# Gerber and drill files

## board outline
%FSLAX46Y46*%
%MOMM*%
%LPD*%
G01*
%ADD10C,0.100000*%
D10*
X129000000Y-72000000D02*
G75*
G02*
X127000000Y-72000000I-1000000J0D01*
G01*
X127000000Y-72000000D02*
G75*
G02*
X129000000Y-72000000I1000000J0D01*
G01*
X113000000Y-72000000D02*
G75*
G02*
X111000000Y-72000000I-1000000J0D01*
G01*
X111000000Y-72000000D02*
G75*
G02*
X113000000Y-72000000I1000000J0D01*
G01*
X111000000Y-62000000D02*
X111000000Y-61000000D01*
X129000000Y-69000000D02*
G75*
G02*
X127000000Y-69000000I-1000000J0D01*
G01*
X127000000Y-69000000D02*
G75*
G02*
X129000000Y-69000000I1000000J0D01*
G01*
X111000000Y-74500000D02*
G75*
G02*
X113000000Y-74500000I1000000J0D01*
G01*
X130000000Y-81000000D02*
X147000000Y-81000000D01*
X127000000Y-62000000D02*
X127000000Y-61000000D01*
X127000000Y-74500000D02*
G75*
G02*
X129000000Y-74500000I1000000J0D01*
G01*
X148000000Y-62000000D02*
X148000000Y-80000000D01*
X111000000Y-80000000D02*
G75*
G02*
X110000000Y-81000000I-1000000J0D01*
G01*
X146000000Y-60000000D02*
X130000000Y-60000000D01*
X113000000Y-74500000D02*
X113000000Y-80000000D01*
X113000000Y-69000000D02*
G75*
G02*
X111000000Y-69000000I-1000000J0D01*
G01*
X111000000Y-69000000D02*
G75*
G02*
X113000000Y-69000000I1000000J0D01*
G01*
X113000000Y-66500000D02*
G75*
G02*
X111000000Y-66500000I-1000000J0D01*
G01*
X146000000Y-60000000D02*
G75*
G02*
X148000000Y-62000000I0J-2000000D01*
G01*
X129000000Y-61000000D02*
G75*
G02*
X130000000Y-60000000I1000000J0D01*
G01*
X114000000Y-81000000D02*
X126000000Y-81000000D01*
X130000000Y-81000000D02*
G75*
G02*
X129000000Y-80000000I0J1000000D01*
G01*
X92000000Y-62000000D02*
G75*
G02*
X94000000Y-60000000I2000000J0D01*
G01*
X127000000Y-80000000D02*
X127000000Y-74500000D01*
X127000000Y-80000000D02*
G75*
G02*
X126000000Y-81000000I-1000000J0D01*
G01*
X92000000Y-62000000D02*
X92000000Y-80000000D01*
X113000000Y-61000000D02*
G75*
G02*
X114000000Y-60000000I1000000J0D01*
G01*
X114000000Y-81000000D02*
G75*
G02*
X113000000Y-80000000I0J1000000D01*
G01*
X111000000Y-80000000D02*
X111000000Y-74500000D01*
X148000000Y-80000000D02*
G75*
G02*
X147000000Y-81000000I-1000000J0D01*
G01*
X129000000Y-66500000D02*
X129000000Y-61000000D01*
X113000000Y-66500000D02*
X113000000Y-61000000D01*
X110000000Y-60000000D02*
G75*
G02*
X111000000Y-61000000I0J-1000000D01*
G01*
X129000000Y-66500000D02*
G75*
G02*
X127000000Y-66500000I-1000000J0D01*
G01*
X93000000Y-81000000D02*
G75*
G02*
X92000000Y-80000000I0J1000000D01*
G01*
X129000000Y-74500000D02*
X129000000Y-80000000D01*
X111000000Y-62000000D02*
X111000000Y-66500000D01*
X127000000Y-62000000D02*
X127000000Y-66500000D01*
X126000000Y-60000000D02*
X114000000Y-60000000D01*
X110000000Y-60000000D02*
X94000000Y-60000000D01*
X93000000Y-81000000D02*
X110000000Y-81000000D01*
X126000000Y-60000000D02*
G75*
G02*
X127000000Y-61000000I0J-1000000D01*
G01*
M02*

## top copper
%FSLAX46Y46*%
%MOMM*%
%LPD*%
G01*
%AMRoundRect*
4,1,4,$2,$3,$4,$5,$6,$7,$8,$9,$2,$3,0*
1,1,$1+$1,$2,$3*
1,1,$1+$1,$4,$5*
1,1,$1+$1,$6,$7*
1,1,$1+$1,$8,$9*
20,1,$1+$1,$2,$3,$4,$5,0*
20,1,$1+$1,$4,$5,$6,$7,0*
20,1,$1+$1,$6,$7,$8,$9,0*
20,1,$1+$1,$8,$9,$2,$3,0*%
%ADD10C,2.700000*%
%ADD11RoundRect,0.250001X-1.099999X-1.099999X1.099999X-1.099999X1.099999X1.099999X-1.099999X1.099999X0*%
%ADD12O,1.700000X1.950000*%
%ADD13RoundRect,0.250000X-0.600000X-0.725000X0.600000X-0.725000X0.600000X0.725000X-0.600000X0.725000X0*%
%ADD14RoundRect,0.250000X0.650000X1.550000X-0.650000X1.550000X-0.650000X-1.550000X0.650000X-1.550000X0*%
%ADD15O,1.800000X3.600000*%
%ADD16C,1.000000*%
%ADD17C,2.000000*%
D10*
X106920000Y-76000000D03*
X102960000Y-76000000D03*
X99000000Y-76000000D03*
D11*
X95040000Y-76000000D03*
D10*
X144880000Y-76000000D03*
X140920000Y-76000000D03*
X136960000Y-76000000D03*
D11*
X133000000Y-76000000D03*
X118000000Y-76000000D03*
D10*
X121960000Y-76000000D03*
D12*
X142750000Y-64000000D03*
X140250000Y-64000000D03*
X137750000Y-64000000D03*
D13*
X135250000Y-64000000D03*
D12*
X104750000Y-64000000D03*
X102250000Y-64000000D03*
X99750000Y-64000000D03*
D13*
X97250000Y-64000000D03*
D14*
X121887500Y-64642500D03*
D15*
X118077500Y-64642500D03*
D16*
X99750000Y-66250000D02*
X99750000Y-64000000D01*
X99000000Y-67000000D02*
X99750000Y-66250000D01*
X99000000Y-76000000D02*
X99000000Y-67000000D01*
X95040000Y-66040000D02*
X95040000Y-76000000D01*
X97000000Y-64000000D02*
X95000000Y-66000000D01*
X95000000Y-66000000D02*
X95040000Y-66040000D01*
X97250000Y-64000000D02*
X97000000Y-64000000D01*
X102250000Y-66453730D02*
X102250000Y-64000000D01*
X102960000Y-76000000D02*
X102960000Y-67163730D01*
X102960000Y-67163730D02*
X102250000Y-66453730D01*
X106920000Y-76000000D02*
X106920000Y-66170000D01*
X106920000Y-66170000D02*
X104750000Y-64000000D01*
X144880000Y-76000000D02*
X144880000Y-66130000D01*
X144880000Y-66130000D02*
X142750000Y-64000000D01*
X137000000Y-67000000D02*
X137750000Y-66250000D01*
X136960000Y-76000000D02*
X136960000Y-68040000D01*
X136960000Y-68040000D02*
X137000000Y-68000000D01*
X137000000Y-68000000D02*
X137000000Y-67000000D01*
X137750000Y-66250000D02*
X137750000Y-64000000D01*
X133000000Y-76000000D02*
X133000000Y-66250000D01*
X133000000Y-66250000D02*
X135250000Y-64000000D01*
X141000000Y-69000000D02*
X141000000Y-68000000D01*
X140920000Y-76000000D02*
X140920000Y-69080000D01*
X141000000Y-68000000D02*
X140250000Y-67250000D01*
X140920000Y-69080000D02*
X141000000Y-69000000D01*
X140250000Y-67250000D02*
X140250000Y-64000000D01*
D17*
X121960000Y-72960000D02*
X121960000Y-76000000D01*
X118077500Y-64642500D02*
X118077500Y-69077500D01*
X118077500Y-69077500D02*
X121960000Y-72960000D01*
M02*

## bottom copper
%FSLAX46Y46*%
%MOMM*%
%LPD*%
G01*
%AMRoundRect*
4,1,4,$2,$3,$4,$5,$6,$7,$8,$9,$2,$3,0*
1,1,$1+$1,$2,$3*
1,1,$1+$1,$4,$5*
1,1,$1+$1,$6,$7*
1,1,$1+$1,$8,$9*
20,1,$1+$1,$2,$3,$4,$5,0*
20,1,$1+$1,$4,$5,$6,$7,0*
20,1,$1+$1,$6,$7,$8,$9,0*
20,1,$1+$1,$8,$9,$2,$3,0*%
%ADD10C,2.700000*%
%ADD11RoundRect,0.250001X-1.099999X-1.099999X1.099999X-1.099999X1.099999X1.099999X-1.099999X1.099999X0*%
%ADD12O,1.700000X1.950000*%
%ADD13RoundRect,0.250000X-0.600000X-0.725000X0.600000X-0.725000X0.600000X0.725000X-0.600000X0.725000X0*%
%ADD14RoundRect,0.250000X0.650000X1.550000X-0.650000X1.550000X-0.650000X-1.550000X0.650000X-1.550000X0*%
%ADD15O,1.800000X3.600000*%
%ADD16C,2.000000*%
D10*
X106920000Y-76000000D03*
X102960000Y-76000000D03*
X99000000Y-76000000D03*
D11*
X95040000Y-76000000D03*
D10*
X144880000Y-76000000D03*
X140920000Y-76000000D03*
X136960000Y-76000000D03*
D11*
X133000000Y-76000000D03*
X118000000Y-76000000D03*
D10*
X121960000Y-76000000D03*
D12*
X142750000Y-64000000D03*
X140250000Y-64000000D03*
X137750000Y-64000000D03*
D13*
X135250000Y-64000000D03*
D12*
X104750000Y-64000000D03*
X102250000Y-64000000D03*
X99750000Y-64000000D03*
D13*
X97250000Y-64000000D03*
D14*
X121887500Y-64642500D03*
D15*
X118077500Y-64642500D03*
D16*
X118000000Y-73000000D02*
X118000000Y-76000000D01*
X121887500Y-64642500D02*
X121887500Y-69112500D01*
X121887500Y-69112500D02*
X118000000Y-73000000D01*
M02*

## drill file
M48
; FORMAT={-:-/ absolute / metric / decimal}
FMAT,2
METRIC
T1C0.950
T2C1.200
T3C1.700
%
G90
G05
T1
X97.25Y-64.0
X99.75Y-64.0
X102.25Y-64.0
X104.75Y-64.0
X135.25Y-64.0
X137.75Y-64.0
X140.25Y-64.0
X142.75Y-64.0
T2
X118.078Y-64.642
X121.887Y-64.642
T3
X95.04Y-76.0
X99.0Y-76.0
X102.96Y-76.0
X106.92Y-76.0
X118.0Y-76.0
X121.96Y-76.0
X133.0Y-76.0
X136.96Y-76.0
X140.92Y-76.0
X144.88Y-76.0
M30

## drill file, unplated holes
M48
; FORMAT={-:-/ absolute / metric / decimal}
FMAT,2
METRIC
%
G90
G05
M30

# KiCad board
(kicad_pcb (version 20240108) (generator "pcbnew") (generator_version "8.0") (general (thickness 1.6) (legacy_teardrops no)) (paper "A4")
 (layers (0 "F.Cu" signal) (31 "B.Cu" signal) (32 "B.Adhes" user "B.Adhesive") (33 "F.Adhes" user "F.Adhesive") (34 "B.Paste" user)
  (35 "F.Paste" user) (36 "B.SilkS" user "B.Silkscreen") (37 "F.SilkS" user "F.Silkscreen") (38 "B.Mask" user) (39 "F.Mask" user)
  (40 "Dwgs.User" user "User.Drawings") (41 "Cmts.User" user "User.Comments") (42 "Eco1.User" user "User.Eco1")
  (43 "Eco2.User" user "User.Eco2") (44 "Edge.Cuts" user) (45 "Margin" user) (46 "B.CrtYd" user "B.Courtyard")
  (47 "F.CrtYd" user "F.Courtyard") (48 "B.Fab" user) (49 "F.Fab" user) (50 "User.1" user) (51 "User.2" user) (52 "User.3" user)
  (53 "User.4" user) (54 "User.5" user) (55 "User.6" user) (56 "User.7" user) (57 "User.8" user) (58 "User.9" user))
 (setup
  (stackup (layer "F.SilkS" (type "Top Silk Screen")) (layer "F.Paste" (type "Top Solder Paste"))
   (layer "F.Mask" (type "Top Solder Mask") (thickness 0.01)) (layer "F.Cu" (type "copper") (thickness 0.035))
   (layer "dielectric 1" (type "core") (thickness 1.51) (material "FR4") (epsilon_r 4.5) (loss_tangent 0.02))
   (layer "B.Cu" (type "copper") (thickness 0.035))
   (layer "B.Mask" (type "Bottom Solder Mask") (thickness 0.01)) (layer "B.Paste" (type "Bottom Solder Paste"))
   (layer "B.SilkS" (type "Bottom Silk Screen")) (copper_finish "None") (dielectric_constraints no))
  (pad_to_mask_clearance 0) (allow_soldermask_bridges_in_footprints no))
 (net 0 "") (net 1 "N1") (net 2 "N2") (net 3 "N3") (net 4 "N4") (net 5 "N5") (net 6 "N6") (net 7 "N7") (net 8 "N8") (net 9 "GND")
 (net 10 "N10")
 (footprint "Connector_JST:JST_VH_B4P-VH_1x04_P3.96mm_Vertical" (layer "F.Cu") (at 95.04 76)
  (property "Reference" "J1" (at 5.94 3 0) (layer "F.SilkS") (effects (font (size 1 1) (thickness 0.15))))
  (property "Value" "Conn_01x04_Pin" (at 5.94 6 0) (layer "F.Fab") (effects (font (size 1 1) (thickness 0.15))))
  (pad "1" thru_hole roundrect (at 0 0) (size 2.7 2.7) (drill 1.7) (layers "*.Cu" "*.Mask") (remove_unused_layers no)
   (roundrect_rratio 0.092593) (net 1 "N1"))
  (pad "2" thru_hole circle (at 3.96 0) (size 2.7 2.7) (drill 1.7) (layers "*.Cu" "*.Mask") (remove_unused_layers no) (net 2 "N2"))
  (pad "3" thru_hole circle (at 7.92 0) (size 2.7 2.7) (drill 1.7) (layers "*.Cu" "*.Mask") (remove_unused_layers no) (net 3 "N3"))
  (pad "4" thru_hole circle (at 11.88 0) (size 2.7 2.7) (drill 1.7) (layers "*.Cu" "*.Mask") (remove_unused_layers no) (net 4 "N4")))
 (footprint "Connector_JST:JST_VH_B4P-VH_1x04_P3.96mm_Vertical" (layer "F.Cu") (at 133 76)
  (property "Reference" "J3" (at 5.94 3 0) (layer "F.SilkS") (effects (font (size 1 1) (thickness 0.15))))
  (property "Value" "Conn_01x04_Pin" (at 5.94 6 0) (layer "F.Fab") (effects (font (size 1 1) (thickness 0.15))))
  (pad "1" thru_hole roundrect (at 0 0) (size 2.7 2.7) (drill 1.7) (layers "*.Cu" "*.Mask") (remove_unused_layers no)
   (roundrect_rratio 0.092593) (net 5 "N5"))
  (pad "2" thru_hole circle (at 3.96 0) (size 2.7 2.7) (drill 1.7) (layers "*.Cu" "*.Mask") (remove_unused_layers no) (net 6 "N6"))
  (pad "3" thru_hole circle (at 7.92 0) (size 2.7 2.7) (drill 1.7) (layers "*.Cu" "*.Mask") (remove_unused_layers no) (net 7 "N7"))
  (pad "4" thru_hole circle (at 11.88 0) (size 2.7 2.7) (drill 1.7) (layers "*.Cu" "*.Mask") (remove_unused_layers no) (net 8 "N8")))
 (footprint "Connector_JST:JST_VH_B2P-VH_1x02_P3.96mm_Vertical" (layer "F.Cu") (at 118 76)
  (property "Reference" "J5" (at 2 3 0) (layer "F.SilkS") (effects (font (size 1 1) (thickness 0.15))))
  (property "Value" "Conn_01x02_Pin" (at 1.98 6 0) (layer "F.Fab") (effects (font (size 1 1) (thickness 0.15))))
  (pad "1" thru_hole roundrect (at 0 0) (size 2.7 2.7) (drill 1.7) (layers "*.Cu" "*.Mask") (remove_unused_layers no)
   (roundrect_rratio 0.092593) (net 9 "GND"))
  (pad "2" thru_hole circle (at 3.96 0) (size 2.7 2.7) (drill 1.7) (layers "*.Cu" "*.Mask") (remove_unused_layers no) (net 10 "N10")))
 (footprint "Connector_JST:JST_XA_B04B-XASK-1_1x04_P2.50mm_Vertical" (layer "B.Cu") (at 135.25 64)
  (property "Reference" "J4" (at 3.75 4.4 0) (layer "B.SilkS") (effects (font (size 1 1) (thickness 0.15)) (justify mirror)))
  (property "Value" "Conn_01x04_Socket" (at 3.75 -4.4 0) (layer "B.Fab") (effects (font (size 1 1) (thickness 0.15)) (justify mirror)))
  (pad "1" thru_hole roundrect (at 0 0) (size 1.7 1.95) (drill 0.95) (layers "*.Cu" "*.Mask") (remove_unused_layers no)
   (roundrect_rratio 0.147059) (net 5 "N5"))
  (pad "2" thru_hole oval (at 2.5 0) (size 1.7 1.95) (drill 0.95) (layers "*.Cu" "*.Mask") (remove_unused_layers no) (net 6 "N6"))
  (pad "3" thru_hole oval (at 5 0) (size 1.7 1.95) (drill 0.95) (layers "*.Cu" "*.Mask") (remove_unused_layers no) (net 7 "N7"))
  (pad "4" thru_hole oval (at 7.5 0) (size 1.7 1.95) (drill 0.95) (layers "*.Cu" "*.Mask") (remove_unused_layers no) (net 8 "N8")))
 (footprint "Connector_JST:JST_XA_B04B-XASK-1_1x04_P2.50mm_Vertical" (layer "B.Cu") (at 97.25 64)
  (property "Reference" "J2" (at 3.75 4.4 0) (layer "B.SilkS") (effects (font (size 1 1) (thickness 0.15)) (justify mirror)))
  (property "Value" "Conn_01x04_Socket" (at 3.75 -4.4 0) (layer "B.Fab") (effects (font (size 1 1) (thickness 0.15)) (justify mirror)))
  (pad "1" thru_hole roundrect (at 0 0) (size 1.7 1.95) (drill 0.95) (layers "*.Cu" "*.Mask") (remove_unused_layers no)
   (roundrect_rratio 0.147059) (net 1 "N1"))
  (pad "2" thru_hole oval (at 2.5 0) (size 1.7 1.95) (drill 0.95) (layers "*.Cu" "*.Mask") (remove_unused_layers no) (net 2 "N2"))
  (pad "3" thru_hole oval (at 5 0) (size 1.7 1.95) (drill 0.95) (layers "*.Cu" "*.Mask") (remove_unused_layers no) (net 3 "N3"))
  (pad "4" thru_hole oval (at 7.5 0) (size 1.7 1.95) (drill 0.95) (layers "*.Cu" "*.Mask") (remove_unused_layers no) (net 4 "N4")))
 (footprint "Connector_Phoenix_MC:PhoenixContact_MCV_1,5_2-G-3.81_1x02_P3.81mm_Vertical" (layer "B.Cu") (at 121.8875 64.6425 180)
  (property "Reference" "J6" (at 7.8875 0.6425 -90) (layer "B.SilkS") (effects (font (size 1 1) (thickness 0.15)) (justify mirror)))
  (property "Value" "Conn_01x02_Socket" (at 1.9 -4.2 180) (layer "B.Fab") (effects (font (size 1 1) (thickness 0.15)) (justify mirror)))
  (pad "1" thru_hole roundrect (at 0 0 180) (size 1.8 3.6) (drill 1.2) (layers "*.Cu" "*.Mask") (remove_unused_layers no)
   (roundrect_rratio 0.138889) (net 9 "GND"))
  (pad "2" thru_hole oval (at 3.81 0 180) (size 1.8 3.6) (drill 1.2) (layers "*.Cu" "*.Mask") (remove_unused_layers no) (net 10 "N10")))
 (gr_line (start 111 62) (end 111 61) (stroke (width 0.1) (type default)) (layer "Edge.Cuts"))
 (gr_circle (center 128 69) (end 129 69) (stroke (width 0.1) (type default)) (fill none) (layer "Edge.Cuts"))
 (gr_arc (start 111 74.5) (mid 112 73.5) (end 113 74.5) (stroke (width 0.1) (type default)) (layer "Edge.Cuts"))
 (gr_line (start 130 81) (end 147 81) (stroke (width 0.1) (type default)) (layer "Edge.Cuts"))
 (gr_line (start 127 62) (end 127 61) (stroke (width 0.1) (type default)) (layer "Edge.Cuts"))
 (gr_arc (start 127 74.5) (mid 128 73.5) (end 129 74.5) (stroke (width 0.1) (type default)) (layer "Edge.Cuts"))
 (gr_line (start 148 62) (end 148 80) (stroke (width 0.1) (type default)) (layer "Edge.Cuts"))
 (gr_arc (start 111 80) (mid 110.707107 80.707107) (end 110 81) (stroke (width 0.1) (type default)) (layer "Edge.Cuts"))
 (gr_line (start 146 60) (end 130 60) (stroke (width 0.1) (type default)) (layer "Edge.Cuts"))
 (gr_line (start 113 74.5) (end 113 80) (stroke (width 0.1) (type default)) (layer "Edge.Cuts"))
 (gr_circle (center 112 69) (end 113 69) (stroke (width 0.1) (type default)) (fill none) (layer "Edge.Cuts"))
 (gr_arc (start 113 66.5) (mid 112 67.5) (end 111 66.5) (stroke (width 0.1) (type default)) (layer "Edge.Cuts"))
 (gr_arc (start 146 60) (mid 147.414214 60.585786) (end 148 62) (stroke (width 0.1) (type default)) (layer "Edge.Cuts"))
 (gr_arc (start 129 61) (mid 129.292893 60.292893) (end 130 60) (stroke (width 0.1) (type default)) (layer "Edge.Cuts"))
 (gr_line (start 114 81) (end 126 81) (stroke (width 0.1) (type default)) (layer "Edge.Cuts"))
 (gr_arc (start 130 81) (mid 129.292893 80.707107) (end 129 80) (stroke (width 0.1) (type default)) (layer "Edge.Cuts"))
 (gr_arc (start 92 62) (mid 92.585786 60.585786) (end 94 60) (stroke (width 0.1) (type default)) (layer "Edge.Cuts"))
 (gr_line (start 127 80) (end 127 74.5) (stroke (width 0.1) (type default)) (layer "Edge.Cuts"))
 (gr_arc (start 127 80) (mid 126.707107 80.707107) (end 126 81) (stroke (width 0.1) (type default)) (layer "Edge.Cuts"))
 (gr_circle (center 112 72) (end 113 72) (stroke (width 0.1) (type default)) (fill none) (layer "Edge.Cuts"))
 (gr_line (start 92 62) (end 92 80) (stroke (width 0.1) (type default)) (layer "Edge.Cuts"))
 (gr_arc (start 113 61) (mid 113.292893 60.292893) (end 114 60) (stroke (width 0.1) (type default)) (layer "Edge.Cuts"))
 (gr_arc (start 114 81) (mid 113.292893 80.707107) (end 113 80) (stroke (width 0.1) (type default)) (layer "Edge.Cuts"))
 (gr_line (start 111 80) (end 111 74.5) (stroke (width 0.1) (type default)) (layer "Edge.Cuts"))
 (gr_arc (start 148 80) (mid 147.707107 80.707107) (end 147 81) (stroke (width 0.1) (type default)) (layer "Edge.Cuts"))
 (gr_line (start 129 66.5) (end 129 61) (stroke (width 0.1) (type default)) (layer "Edge.Cuts"))
 (gr_line (start 113 66.5) (end 113 61) (stroke (width 0.1) (type default)) (layer "Edge.Cuts"))
 (gr_arc (start 110 60) (mid 110.707107 60.292893) (end 111 61) (stroke (width 0.1) (type default)) (layer "Edge.Cuts"))
 (gr_arc (start 129 66.5) (mid 128 67.5) (end 127 66.5) (stroke (width 0.1) (type default)) (layer "Edge.Cuts"))
 (gr_arc (start 93 81) (mid 92.292893 80.707107) (end 92 80) (stroke (width 0.1) (type default)) (layer "Edge.Cuts"))
 (gr_line (start 129 74.5) (end 129 80) (stroke (width 0.1) (type default)) (layer "Edge.Cuts"))
 (gr_line (start 111 62) (end 111 66.5) (stroke (width 0.1) (type default)) (layer "Edge.Cuts"))
 (gr_line (start 127 62) (end 127 66.5) (stroke (width 0.1) (type default)) (layer "Edge.Cuts"))
 (gr_line (start 126 60) (end 114 60) (stroke (width 0.1) (type default)) (layer "Edge.Cuts"))
 (gr_circle (center 128 72) (end 129 72) (stroke (width 0.1) (type default)) (fill none) (layer "Edge.Cuts"))
 (gr_line (start 110 60) (end 94 60) (stroke (width 0.1) (type default)) (layer "Edge.Cuts"))
 (gr_line (start 93 81) (end 110 81) (stroke (width 0.1) (type default)) (layer "Edge.Cuts"))
 (gr_arc (start 126 60) (mid 126.707107 60.292893) (end 127 61) (stroke (width 0.1) (type default)) (layer "Edge.Cuts"))
 (segment (start 99.75 66.25) (end 99.75 64) (width 1) (layer "F.Cu") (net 2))
 (segment (start 99 67) (end 99.75 66.25) (width 1) (layer "F.Cu") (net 2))
 (segment (start 99 76) (end 99 67) (width 1) (layer "F.Cu") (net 2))
 (segment (start 95.04 66.04) (end 95.04 76) (width 1) (layer "F.Cu") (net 1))
 (segment (start 97 64) (end 95 66) (width 1) (layer "F.Cu") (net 1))
 (segment (start 95 66) (end 95.04 66.04) (width 1) (layer "F.Cu") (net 1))
 (segment (start 97.25 64) (end 97 64) (width 1) (layer "F.Cu") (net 1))
 (segment (start 102.25 66.45373) (end 102.25 64) (width 1) (layer "F.Cu") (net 3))
 (segment (start 102.96 76) (end 102.96 67.16373) (width 1) (layer "F.Cu") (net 3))
 (segment (start 102.96 67.16373) (end 102.25 66.45373) (width 1) (layer "F.Cu") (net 3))
 (segment (start 106.92 76) (end 106.92 66.17) (width 1) (layer "F.Cu") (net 4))
 (segment (start 106.92 66.17) (end 104.75 64) (width 1) (layer "F.Cu") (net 4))
 (segment (start 144.88 76) (end 144.88 66.13) (width 1) (layer "F.Cu") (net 8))
 (segment (start 144.88 66.13) (end 142.75 64) (width 1) (layer "F.Cu") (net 8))
 (segment (start 137 67) (end 137.75 66.25) (width 1) (layer "F.Cu") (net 6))
 (segment (start 136.96 76) (end 136.96 68.04) (width 1) (layer "F.Cu") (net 6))
 (segment (start 136.96 68.04) (end 137 68) (width 1) (layer "F.Cu") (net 6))
 (segment (start 137 68) (end 137 67) (width 1) (layer "F.Cu") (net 6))
 (segment (start 137.75 66.25) (end 137.75 64) (width 1) (layer "F.Cu") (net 6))
 (segment (start 133 76) (end 133 66.25) (width 1) (layer "F.Cu") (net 5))
 (segment (start 133 66.25) (end 135.25 64) (width 1) (layer "F.Cu") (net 5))
 (segment (start 141 69) (end 141 68) (width 1) (layer "F.Cu") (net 7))
 (segment (start 140.92 76) (end 140.92 69.08) (width 1) (layer "F.Cu") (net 7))
 (segment (start 141 68) (end 140.25 67.25) (width 1) (layer "F.Cu") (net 7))
 (segment (start 140.92 69.08) (end 141 69) (width 1) (layer "F.Cu") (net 7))
 (segment (start 140.25 67.25) (end 140.25 64) (width 1) (layer "F.Cu") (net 7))
 (segment (start 121.96 72.96) (end 121.96 76) (width 2) (layer "F.Cu") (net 10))
 (segment (start 118.0775 64.6425) (end 118.0775 69.0775) (width 2) (layer "F.Cu") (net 10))
 (segment (start 118.0775 69.0775) (end 121.96 72.96) (width 2) (layer "F.Cu") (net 10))
 (segment (start 118 73) (end 118 76) (width 2) (layer "B.Cu") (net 9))
 (segment (start 121.8875 64.6425) (end 121.8875 69.1125) (width 2) (layer "B.Cu") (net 9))
 (segment (start 121.8875 69.1125) (end 118 73) (width 2) (layer "B.Cu") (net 9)))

